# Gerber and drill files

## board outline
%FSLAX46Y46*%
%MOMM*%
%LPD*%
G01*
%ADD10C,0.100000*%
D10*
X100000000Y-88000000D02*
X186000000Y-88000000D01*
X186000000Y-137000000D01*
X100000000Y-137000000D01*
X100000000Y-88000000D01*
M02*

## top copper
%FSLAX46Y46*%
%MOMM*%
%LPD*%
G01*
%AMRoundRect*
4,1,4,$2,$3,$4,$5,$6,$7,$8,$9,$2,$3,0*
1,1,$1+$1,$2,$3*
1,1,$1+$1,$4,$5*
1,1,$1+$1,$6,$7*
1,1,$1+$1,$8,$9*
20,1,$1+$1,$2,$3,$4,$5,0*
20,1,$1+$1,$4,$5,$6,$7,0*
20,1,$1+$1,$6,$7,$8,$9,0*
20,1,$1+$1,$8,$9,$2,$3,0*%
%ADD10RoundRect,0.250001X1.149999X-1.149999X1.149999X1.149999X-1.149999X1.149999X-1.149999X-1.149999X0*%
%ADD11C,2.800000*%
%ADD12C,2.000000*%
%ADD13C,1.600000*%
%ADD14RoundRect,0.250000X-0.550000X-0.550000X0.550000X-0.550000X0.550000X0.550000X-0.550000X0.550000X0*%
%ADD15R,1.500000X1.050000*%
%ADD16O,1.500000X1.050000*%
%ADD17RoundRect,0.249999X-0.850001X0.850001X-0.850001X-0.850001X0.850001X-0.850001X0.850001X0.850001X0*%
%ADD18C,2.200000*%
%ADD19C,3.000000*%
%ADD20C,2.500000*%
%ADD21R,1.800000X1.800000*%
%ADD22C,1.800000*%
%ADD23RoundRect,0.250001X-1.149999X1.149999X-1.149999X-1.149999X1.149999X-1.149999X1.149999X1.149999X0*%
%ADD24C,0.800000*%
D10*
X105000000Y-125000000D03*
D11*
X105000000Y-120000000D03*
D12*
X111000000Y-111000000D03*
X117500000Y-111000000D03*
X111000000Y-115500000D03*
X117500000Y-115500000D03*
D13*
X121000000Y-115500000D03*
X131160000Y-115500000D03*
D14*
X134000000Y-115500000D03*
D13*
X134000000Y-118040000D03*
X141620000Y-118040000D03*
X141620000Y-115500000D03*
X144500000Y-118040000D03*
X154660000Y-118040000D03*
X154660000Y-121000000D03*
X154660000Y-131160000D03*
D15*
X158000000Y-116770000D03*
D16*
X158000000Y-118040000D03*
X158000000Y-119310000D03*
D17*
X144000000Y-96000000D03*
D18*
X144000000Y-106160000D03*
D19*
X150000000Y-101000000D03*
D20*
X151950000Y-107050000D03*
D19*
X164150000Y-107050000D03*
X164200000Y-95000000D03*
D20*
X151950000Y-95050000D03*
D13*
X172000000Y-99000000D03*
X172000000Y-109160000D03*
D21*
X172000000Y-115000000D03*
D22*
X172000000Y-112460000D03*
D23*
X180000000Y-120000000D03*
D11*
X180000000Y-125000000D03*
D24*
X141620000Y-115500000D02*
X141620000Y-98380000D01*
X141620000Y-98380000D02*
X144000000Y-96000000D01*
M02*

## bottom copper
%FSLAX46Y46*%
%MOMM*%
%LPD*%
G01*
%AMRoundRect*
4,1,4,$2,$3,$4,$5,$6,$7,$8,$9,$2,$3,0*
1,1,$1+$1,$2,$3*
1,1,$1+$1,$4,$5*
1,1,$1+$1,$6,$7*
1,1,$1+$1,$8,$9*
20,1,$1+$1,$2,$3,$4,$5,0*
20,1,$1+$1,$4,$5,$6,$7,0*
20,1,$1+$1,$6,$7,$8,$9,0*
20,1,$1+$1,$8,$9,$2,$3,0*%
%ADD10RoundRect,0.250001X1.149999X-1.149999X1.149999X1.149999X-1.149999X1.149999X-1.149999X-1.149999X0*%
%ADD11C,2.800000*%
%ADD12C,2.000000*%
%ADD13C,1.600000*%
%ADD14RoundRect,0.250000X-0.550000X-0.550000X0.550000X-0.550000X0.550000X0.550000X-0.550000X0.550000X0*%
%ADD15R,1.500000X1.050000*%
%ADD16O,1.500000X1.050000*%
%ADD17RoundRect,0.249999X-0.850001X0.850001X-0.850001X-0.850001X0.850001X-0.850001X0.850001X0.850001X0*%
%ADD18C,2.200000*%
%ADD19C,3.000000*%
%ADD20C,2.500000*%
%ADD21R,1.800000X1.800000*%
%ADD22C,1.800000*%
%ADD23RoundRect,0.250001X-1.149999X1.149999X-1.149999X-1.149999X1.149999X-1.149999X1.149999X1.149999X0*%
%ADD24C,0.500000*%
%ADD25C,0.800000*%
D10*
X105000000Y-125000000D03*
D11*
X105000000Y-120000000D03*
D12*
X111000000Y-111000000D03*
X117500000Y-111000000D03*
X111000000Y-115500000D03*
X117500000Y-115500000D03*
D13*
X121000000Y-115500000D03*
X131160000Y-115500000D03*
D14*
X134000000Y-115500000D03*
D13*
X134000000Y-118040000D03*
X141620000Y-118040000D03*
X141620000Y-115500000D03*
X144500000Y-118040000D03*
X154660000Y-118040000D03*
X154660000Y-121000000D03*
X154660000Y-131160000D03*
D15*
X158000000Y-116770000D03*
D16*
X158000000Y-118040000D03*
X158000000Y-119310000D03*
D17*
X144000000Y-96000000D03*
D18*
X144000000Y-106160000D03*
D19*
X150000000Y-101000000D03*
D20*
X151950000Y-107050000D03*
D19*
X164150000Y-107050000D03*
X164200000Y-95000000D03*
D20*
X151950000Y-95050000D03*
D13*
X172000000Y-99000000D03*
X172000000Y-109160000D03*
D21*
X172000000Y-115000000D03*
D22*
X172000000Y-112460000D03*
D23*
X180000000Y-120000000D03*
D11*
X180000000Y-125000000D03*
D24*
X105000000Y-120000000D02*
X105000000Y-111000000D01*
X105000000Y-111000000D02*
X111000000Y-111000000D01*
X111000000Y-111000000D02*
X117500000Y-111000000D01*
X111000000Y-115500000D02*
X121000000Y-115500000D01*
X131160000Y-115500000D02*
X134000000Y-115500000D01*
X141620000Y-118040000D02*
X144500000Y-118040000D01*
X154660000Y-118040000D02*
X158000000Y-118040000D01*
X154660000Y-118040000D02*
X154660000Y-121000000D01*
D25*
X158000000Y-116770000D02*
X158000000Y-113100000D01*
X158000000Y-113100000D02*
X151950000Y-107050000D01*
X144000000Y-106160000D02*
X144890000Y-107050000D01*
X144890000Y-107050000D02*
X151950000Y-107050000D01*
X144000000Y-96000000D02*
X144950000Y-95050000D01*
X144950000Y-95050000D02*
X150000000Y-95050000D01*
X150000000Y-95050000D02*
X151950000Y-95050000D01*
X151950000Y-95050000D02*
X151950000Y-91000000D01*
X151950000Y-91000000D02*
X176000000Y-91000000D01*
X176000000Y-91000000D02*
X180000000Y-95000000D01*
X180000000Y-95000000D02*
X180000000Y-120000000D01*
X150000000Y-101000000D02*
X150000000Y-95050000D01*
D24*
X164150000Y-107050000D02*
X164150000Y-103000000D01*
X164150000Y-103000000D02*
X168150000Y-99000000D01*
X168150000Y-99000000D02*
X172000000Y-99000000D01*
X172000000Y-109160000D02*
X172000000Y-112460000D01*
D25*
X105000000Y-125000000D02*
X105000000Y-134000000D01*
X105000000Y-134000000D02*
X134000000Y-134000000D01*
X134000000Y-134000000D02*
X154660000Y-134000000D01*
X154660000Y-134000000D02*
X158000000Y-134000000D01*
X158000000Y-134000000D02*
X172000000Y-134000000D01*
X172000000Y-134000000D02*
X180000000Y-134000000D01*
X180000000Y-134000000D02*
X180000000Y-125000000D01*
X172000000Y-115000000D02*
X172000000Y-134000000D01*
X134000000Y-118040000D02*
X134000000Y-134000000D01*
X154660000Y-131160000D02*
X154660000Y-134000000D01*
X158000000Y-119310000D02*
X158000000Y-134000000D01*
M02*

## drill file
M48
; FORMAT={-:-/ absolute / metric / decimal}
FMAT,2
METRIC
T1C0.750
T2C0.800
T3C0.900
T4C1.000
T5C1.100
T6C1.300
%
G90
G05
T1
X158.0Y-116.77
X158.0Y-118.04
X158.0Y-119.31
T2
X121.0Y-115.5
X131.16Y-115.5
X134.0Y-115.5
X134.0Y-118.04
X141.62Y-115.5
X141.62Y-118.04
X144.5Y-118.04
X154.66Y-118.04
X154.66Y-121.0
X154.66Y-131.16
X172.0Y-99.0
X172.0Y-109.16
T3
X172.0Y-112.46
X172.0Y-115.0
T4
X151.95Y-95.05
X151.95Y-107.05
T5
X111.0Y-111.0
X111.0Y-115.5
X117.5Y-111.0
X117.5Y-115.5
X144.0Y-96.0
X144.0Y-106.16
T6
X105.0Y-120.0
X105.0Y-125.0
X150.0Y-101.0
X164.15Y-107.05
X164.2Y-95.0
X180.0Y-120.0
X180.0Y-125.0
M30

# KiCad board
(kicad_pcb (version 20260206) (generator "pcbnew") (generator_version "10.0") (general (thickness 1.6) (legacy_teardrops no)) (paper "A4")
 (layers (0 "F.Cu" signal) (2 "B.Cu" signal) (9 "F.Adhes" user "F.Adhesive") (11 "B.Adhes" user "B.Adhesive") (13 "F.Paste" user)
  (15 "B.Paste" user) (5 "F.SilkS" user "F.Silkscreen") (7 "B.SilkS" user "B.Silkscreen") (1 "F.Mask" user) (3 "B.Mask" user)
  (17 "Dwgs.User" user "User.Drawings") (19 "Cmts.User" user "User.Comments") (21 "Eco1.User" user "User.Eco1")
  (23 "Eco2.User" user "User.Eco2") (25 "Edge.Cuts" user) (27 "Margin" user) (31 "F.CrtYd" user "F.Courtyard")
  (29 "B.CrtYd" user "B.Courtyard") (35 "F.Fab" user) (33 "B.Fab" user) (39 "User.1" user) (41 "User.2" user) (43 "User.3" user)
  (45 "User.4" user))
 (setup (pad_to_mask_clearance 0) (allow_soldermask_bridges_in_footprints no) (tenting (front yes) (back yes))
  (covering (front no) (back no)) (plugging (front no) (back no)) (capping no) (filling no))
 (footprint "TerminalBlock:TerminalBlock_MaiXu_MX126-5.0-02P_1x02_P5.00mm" (layer "F.Cu") (at 105 125 90)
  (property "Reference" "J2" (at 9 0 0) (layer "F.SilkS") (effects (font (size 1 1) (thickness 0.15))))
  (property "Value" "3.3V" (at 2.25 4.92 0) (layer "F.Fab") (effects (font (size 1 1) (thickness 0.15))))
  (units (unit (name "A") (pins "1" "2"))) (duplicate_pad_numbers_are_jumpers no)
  (pad "1" thru_hole roundrect (at 0 0 90) (size 2.8 2.8) (drill 1.3) (layers "*.Cu" "*.Mask") (remove_unused_layers no)
   (roundrect_rratio 0.089286) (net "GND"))
  (pad "2" thru_hole circle (at 5 0 90) (size 2.8 2.8) (drill 1.3) (layers "*.Cu" "*.Mask") (remove_unused_layers no) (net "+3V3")))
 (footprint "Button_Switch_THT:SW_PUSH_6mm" (layer "F.Cu") (at 111 111)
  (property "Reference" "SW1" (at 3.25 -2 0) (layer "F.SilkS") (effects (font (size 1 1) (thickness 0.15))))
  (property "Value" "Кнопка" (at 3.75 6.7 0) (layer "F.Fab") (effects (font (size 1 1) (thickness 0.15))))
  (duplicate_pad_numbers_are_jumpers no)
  (pad "1" thru_hole circle (at 0 0 90) (size 2 2) (drill 1.1) (layers "*.Cu" "*.Mask") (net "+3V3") (remove_unused_layers no))
  (pad "1" thru_hole circle (at 6.5 0 90) (size 2 2) (drill 1.1) (layers "*.Cu" "*.Mask") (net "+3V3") (remove_unused_layers no))
  (pad "2" thru_hole circle (at 0 4.5 90) (size 2 2) (drill 1.1) (layers "*.Cu" "*.Mask") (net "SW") (remove_unused_layers no))
  (pad "2" thru_hole circle (at 6.5 4.5 90) (size 2 2) (drill 1.1) (layers "*.Cu" "*.Mask") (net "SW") (remove_unused_layers no)))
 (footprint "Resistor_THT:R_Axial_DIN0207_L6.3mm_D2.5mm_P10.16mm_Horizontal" (layer "F.Cu") (at 121 115.5)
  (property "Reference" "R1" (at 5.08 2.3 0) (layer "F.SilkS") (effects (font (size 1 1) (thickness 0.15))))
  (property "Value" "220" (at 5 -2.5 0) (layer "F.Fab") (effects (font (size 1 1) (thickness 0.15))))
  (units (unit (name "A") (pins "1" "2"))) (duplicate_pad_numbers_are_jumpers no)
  (pad "1" thru_hole circle (at 0 0) (size 1.6 1.6) (drill 0.8) (layers "*.Cu" "*.Mask") (remove_unused_layers no) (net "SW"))
  (pad "2" thru_hole circle (at 10.16 0) (size 1.6 1.6) (drill 0.8) (layers "*.Cu" "*.Mask") (remove_unused_layers no) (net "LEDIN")))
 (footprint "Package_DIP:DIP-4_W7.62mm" (layer "F.Cu") (at 134 115.5)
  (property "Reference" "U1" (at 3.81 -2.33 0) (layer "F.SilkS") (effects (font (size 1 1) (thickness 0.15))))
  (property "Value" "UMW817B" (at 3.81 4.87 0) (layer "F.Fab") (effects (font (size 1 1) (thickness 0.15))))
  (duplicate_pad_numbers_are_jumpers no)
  (pad "1" thru_hole roundrect (at 0 0) (size 1.6 1.6) (drill 0.8) (layers "*.Cu" "*.Mask") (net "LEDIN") (remove_unused_layers no)
   (roundrect_rratio 0.15625))
  (pad "2" thru_hole circle (at 0 2.54) (size 1.6 1.6) (drill 0.8) (layers "*.Cu" "*.Mask") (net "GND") (remove_unused_layers no))
  (pad "3" thru_hole circle (at 7.62 2.54) (size 1.6 1.6) (drill 0.8) (layers "*.Cu" "*.Mask") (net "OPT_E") (remove_unused_layers no))
  (pad "4" thru_hole circle (at 7.62 0) (size 1.6 1.6) (drill 0.8) (layers "*.Cu" "*.Mask") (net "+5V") (remove_unused_layers no))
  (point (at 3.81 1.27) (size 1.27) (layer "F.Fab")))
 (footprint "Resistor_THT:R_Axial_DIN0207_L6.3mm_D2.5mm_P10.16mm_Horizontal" (layer "F.Cu") (at 144.5 118.04)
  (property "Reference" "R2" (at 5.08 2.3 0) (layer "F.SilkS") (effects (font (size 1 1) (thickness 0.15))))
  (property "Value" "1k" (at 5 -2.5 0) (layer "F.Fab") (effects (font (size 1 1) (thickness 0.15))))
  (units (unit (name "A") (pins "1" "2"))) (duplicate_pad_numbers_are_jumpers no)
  (pad "1" thru_hole circle (at 0 0) (size 1.6 1.6) (drill 0.8) (layers "*.Cu" "*.Mask") (remove_unused_layers no) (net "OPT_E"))
  (pad "2" thru_hole circle (at 10.16 0) (size 1.6 1.6) (drill 0.8) (layers "*.Cu" "*.Mask") (remove_unused_layers no) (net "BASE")))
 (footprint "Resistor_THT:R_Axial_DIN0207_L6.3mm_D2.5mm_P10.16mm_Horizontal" (layer "F.Cu") (at 154.66 121 -90)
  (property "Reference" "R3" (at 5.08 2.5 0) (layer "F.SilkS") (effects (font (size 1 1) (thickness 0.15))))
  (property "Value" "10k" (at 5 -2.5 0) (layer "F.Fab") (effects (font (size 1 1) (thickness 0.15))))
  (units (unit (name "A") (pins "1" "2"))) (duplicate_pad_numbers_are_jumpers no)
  (pad "1" thru_hole circle (at 0 0 270) (size 1.6 1.6) (drill 0.8) (layers "*.Cu" "*.Mask") (remove_unused_layers no) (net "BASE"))
  (pad "2" thru_hole circle (at 10.16 0 270) (size 1.6 1.6) (drill 0.8) (layers "*.Cu" "*.Mask") (remove_unused_layers no) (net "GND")))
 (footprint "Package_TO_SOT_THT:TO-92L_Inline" (layer "F.Cu") (at 158 116.77 -90)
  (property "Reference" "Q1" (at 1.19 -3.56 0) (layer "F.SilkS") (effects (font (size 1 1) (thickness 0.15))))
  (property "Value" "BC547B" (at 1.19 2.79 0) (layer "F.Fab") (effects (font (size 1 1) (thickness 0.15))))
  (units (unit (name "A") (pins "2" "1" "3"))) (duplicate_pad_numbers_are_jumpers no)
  (pad "1" thru_hole rect (at 0 0 270) (size 1.05 1.5) (drill 0.75) (layers "*.Cu" "*.Mask") (remove_unused_layers no) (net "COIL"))
  (pad "2" thru_hole oval (at 1.27 0 270) (size 1.05 1.5) (drill 0.75) (layers "*.Cu" "*.Mask") (remove_unused_layers no) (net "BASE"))
  (pad "3" thru_hole oval (at 2.54 0 270) (size 1.05 1.5) (drill 0.75) (layers "*.Cu" "*.Mask") (remove_unused_layers no) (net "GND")))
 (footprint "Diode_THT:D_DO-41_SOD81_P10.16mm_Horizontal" (layer "F.Cu") (at 144 96 -90)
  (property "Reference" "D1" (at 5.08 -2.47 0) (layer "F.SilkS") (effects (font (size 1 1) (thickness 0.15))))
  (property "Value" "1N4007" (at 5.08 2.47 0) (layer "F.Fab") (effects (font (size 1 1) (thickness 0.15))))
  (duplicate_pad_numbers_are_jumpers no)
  (pad "1" thru_hole roundrect (at 0 0 270) (size 2.2 2.2) (drill 1.1) (layers "*.Cu" "*.Mask") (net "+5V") (remove_unused_layers no)
   (roundrect_rratio 0.113636))
  (pad "2" thru_hole circle (at 10.16 0 270) (size 2.2 2.2) (drill 1.1) (layers "*.Cu" "*.Mask") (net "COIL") (remove_unused_layers no)))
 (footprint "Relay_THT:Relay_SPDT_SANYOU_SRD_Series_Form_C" (layer "F.Cu") (at 150 101)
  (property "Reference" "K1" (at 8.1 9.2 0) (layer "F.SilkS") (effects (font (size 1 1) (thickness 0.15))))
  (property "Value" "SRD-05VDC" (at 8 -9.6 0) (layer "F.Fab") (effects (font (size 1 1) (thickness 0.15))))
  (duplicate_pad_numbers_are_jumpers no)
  (pad "1" thru_hole circle (at 0 0 90) (size 3 3) (drill 1.3) (layers "*.Cu" "*.Mask") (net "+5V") (remove_unused_layers no))
  (pad "2" thru_hole circle (at 1.95 6.05 90) (size 2.5 2.5) (drill 1) (layers "*.Cu" "*.Mask") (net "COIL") (remove_unused_layers no))
  (pad "3" thru_hole circle (at 14.15 6.05 90) (size 3 3) (drill 1.3) (layers "*.Cu" "*.Mask") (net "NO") (remove_unused_layers no))
  (pad "4" thru_hole circle (at 14.2 -6 90) (size 3 3) (drill 1.3) (layers "*.Cu" "*.Mask") (remove_unused_layers no))
  (pad "5" thru_hole circle (at 1.95 -5.95 90) (size 2.5 2.5) (drill 1) (layers "*.Cu" "*.Mask") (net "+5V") (remove_unused_layers no)))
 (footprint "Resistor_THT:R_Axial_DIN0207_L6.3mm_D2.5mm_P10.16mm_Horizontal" (layer "F.Cu") (at 172 99 -90)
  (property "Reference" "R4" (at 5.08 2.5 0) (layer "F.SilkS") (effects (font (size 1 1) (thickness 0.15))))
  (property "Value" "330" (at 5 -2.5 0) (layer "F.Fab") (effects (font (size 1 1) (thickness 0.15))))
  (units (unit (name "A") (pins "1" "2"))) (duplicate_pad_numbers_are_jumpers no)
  (pad "1" thru_hole circle (at 0 0 270) (size 1.6 1.6) (drill 0.8) (layers "*.Cu" "*.Mask") (remove_unused_layers no) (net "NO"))
  (pad "2" thru_hole circle (at 10.16 0 270) (size 1.6 1.6) (drill 0.8) (layers "*.Cu" "*.Mask") (remove_unused_layers no) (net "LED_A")))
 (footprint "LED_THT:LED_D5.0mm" (layer "F.Cu") (at 172 115 90)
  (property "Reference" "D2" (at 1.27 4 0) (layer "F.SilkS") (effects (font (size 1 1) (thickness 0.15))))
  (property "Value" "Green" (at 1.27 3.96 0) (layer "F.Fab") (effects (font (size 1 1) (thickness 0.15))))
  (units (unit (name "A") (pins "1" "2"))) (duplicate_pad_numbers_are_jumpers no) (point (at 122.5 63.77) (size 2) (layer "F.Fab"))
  (pad "1" thru_hole rect (at 0 0 90) (size 1.8 1.8) (drill 0.9) (layers "*.Cu" "*.Mask") (remove_unused_layers no) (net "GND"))
  (pad "2" thru_hole circle (at 2.54 0 90) (size 1.8 1.8) (drill 0.9) (layers "*.Cu" "*.Mask") (remove_unused_layers no) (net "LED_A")))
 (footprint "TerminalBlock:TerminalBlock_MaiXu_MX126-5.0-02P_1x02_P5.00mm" (layer "F.Cu") (at 180 120 -90)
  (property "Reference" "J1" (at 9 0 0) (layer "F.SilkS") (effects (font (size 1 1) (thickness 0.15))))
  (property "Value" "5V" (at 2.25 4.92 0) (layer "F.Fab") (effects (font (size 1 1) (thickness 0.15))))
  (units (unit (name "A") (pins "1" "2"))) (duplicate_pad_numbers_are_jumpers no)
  (pad "1" thru_hole roundrect (at 0 0 270) (size 2.8 2.8) (drill 1.3) (layers "*.Cu" "*.Mask") (remove_unused_layers no)
   (roundrect_rratio 0.089286) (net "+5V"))
  (pad "2" thru_hole circle (at 5 0 270) (size 2.8 2.8) (drill 1.3) (layers "*.Cu" "*.Mask") (remove_unused_layers no) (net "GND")))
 (gr_rect (start 100 88) (end 186 137) (stroke (width 0.1) (type default)) (fill no) (layer "Edge.Cuts"))
 (segment (start 105 120) (end 105 111) (width 0.5) (layer "B.Cu") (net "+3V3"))
 (segment (start 105 111) (end 111 111) (width 0.5) (layer "B.Cu") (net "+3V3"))
 (segment (start 111 111) (end 117.5 111) (width 0.5) (layer "B.Cu") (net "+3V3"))
 (segment (start 111 115.5) (end 121 115.5) (width 0.5) (layer "B.Cu") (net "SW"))
 (segment (start 131.16 115.5) (end 134 115.5) (width 0.5) (layer "B.Cu") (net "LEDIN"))
 (segment (start 141.62 118.04) (end 144.5 118.04) (width 0.5) (layer "B.Cu") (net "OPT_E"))
 (segment (start 154.66 118.04) (end 158 118.04) (width 0.5) (layer "B.Cu") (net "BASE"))
 (segment (start 154.66 118.04) (end 154.66 121) (width 0.5) (layer "B.Cu") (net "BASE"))
 (segment (start 158 116.77) (end 158 113.1) (width 0.8) (layer "B.Cu") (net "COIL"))
 (segment (start 158 113.1) (end 151.95 107.05) (width 0.8) (layer "B.Cu") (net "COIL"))
 (segment (start 144 106.16) (end 144.89 107.05) (width 0.8) (layer "B.Cu") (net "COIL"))
 (segment (start 144.89 107.05) (end 151.95 107.05) (width 0.8) (layer "B.Cu") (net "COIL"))
 (segment (start 144 96) (end 144.95 95.05) (width 0.8) (layer "B.Cu") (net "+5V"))
 (segment (start 144.95 95.05) (end 150 95.05) (width 0.8) (layer "B.Cu") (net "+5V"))
 (segment (start 150 95.05) (end 151.95 95.05) (width 0.8) (layer "B.Cu") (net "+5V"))
 (segment (start 151.95 95.05) (end 151.95 91) (width 0.8) (layer "B.Cu") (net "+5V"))
 (segment (start 151.95 91) (end 176 91) (width 0.8) (layer "B.Cu") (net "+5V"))
 (segment (start 176 91) (end 180 95) (width 0.8) (layer "B.Cu") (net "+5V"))
 (segment (start 180 95) (end 180 120) (width 0.8) (layer "B.Cu") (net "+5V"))
 (segment (start 150 101) (end 150 95.05) (width 0.8) (layer "B.Cu") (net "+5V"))
 (segment (start 141.62 115.5) (end 141.62 98.38) (width 0.8) (layer "F.Cu") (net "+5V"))
 (segment (start 141.62 98.38) (end 144 96) (width 0.8) (layer "F.Cu") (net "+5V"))
 (segment (start 164.15 107.05) (end 164.15 103) (width 0.5) (layer "B.Cu") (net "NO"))
 (segment (start 164.15 103) (end 168.15 99) (width 0.5) (layer "B.Cu") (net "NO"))
 (segment (start 168.15 99) (end 172 99) (width 0.5) (layer "B.Cu") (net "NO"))
 (segment (start 172 109.16) (end 172 112.46) (width 0.5) (layer "B.Cu") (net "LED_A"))
 (segment (start 105 125) (end 105 134) (width 0.8) (layer "B.Cu") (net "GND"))
 (segment (start 105 134) (end 134 134) (width 0.8) (layer "B.Cu") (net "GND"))
 (segment (start 134 134) (end 154.66 134) (width 0.8) (layer "B.Cu") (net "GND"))
 (segment (start 154.66 134) (end 158 134) (width 0.8) (layer "B.Cu") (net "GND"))
 (segment (start 158 134) (end 172 134) (width 0.8) (layer "B.Cu") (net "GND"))
 (segment (start 172 134) (end 180 134) (width 0.8) (layer "B.Cu") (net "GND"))
 (segment (start 180 134) (end 180 125) (width 0.8) (layer "B.Cu") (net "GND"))
 (segment (start 172 115) (end 172 134) (width 0.8) (layer "B.Cu") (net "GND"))
 (segment (start 134 118.04) (end 134 134) (width 0.8) (layer "B.Cu") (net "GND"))
 (segment (start 154.66 131.16) (end 154.66 134) (width 0.8) (layer "B.Cu") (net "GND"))
 (segment (start 158 119.31) (end 158 134) (width 0.8) (layer "B.Cu") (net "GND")))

